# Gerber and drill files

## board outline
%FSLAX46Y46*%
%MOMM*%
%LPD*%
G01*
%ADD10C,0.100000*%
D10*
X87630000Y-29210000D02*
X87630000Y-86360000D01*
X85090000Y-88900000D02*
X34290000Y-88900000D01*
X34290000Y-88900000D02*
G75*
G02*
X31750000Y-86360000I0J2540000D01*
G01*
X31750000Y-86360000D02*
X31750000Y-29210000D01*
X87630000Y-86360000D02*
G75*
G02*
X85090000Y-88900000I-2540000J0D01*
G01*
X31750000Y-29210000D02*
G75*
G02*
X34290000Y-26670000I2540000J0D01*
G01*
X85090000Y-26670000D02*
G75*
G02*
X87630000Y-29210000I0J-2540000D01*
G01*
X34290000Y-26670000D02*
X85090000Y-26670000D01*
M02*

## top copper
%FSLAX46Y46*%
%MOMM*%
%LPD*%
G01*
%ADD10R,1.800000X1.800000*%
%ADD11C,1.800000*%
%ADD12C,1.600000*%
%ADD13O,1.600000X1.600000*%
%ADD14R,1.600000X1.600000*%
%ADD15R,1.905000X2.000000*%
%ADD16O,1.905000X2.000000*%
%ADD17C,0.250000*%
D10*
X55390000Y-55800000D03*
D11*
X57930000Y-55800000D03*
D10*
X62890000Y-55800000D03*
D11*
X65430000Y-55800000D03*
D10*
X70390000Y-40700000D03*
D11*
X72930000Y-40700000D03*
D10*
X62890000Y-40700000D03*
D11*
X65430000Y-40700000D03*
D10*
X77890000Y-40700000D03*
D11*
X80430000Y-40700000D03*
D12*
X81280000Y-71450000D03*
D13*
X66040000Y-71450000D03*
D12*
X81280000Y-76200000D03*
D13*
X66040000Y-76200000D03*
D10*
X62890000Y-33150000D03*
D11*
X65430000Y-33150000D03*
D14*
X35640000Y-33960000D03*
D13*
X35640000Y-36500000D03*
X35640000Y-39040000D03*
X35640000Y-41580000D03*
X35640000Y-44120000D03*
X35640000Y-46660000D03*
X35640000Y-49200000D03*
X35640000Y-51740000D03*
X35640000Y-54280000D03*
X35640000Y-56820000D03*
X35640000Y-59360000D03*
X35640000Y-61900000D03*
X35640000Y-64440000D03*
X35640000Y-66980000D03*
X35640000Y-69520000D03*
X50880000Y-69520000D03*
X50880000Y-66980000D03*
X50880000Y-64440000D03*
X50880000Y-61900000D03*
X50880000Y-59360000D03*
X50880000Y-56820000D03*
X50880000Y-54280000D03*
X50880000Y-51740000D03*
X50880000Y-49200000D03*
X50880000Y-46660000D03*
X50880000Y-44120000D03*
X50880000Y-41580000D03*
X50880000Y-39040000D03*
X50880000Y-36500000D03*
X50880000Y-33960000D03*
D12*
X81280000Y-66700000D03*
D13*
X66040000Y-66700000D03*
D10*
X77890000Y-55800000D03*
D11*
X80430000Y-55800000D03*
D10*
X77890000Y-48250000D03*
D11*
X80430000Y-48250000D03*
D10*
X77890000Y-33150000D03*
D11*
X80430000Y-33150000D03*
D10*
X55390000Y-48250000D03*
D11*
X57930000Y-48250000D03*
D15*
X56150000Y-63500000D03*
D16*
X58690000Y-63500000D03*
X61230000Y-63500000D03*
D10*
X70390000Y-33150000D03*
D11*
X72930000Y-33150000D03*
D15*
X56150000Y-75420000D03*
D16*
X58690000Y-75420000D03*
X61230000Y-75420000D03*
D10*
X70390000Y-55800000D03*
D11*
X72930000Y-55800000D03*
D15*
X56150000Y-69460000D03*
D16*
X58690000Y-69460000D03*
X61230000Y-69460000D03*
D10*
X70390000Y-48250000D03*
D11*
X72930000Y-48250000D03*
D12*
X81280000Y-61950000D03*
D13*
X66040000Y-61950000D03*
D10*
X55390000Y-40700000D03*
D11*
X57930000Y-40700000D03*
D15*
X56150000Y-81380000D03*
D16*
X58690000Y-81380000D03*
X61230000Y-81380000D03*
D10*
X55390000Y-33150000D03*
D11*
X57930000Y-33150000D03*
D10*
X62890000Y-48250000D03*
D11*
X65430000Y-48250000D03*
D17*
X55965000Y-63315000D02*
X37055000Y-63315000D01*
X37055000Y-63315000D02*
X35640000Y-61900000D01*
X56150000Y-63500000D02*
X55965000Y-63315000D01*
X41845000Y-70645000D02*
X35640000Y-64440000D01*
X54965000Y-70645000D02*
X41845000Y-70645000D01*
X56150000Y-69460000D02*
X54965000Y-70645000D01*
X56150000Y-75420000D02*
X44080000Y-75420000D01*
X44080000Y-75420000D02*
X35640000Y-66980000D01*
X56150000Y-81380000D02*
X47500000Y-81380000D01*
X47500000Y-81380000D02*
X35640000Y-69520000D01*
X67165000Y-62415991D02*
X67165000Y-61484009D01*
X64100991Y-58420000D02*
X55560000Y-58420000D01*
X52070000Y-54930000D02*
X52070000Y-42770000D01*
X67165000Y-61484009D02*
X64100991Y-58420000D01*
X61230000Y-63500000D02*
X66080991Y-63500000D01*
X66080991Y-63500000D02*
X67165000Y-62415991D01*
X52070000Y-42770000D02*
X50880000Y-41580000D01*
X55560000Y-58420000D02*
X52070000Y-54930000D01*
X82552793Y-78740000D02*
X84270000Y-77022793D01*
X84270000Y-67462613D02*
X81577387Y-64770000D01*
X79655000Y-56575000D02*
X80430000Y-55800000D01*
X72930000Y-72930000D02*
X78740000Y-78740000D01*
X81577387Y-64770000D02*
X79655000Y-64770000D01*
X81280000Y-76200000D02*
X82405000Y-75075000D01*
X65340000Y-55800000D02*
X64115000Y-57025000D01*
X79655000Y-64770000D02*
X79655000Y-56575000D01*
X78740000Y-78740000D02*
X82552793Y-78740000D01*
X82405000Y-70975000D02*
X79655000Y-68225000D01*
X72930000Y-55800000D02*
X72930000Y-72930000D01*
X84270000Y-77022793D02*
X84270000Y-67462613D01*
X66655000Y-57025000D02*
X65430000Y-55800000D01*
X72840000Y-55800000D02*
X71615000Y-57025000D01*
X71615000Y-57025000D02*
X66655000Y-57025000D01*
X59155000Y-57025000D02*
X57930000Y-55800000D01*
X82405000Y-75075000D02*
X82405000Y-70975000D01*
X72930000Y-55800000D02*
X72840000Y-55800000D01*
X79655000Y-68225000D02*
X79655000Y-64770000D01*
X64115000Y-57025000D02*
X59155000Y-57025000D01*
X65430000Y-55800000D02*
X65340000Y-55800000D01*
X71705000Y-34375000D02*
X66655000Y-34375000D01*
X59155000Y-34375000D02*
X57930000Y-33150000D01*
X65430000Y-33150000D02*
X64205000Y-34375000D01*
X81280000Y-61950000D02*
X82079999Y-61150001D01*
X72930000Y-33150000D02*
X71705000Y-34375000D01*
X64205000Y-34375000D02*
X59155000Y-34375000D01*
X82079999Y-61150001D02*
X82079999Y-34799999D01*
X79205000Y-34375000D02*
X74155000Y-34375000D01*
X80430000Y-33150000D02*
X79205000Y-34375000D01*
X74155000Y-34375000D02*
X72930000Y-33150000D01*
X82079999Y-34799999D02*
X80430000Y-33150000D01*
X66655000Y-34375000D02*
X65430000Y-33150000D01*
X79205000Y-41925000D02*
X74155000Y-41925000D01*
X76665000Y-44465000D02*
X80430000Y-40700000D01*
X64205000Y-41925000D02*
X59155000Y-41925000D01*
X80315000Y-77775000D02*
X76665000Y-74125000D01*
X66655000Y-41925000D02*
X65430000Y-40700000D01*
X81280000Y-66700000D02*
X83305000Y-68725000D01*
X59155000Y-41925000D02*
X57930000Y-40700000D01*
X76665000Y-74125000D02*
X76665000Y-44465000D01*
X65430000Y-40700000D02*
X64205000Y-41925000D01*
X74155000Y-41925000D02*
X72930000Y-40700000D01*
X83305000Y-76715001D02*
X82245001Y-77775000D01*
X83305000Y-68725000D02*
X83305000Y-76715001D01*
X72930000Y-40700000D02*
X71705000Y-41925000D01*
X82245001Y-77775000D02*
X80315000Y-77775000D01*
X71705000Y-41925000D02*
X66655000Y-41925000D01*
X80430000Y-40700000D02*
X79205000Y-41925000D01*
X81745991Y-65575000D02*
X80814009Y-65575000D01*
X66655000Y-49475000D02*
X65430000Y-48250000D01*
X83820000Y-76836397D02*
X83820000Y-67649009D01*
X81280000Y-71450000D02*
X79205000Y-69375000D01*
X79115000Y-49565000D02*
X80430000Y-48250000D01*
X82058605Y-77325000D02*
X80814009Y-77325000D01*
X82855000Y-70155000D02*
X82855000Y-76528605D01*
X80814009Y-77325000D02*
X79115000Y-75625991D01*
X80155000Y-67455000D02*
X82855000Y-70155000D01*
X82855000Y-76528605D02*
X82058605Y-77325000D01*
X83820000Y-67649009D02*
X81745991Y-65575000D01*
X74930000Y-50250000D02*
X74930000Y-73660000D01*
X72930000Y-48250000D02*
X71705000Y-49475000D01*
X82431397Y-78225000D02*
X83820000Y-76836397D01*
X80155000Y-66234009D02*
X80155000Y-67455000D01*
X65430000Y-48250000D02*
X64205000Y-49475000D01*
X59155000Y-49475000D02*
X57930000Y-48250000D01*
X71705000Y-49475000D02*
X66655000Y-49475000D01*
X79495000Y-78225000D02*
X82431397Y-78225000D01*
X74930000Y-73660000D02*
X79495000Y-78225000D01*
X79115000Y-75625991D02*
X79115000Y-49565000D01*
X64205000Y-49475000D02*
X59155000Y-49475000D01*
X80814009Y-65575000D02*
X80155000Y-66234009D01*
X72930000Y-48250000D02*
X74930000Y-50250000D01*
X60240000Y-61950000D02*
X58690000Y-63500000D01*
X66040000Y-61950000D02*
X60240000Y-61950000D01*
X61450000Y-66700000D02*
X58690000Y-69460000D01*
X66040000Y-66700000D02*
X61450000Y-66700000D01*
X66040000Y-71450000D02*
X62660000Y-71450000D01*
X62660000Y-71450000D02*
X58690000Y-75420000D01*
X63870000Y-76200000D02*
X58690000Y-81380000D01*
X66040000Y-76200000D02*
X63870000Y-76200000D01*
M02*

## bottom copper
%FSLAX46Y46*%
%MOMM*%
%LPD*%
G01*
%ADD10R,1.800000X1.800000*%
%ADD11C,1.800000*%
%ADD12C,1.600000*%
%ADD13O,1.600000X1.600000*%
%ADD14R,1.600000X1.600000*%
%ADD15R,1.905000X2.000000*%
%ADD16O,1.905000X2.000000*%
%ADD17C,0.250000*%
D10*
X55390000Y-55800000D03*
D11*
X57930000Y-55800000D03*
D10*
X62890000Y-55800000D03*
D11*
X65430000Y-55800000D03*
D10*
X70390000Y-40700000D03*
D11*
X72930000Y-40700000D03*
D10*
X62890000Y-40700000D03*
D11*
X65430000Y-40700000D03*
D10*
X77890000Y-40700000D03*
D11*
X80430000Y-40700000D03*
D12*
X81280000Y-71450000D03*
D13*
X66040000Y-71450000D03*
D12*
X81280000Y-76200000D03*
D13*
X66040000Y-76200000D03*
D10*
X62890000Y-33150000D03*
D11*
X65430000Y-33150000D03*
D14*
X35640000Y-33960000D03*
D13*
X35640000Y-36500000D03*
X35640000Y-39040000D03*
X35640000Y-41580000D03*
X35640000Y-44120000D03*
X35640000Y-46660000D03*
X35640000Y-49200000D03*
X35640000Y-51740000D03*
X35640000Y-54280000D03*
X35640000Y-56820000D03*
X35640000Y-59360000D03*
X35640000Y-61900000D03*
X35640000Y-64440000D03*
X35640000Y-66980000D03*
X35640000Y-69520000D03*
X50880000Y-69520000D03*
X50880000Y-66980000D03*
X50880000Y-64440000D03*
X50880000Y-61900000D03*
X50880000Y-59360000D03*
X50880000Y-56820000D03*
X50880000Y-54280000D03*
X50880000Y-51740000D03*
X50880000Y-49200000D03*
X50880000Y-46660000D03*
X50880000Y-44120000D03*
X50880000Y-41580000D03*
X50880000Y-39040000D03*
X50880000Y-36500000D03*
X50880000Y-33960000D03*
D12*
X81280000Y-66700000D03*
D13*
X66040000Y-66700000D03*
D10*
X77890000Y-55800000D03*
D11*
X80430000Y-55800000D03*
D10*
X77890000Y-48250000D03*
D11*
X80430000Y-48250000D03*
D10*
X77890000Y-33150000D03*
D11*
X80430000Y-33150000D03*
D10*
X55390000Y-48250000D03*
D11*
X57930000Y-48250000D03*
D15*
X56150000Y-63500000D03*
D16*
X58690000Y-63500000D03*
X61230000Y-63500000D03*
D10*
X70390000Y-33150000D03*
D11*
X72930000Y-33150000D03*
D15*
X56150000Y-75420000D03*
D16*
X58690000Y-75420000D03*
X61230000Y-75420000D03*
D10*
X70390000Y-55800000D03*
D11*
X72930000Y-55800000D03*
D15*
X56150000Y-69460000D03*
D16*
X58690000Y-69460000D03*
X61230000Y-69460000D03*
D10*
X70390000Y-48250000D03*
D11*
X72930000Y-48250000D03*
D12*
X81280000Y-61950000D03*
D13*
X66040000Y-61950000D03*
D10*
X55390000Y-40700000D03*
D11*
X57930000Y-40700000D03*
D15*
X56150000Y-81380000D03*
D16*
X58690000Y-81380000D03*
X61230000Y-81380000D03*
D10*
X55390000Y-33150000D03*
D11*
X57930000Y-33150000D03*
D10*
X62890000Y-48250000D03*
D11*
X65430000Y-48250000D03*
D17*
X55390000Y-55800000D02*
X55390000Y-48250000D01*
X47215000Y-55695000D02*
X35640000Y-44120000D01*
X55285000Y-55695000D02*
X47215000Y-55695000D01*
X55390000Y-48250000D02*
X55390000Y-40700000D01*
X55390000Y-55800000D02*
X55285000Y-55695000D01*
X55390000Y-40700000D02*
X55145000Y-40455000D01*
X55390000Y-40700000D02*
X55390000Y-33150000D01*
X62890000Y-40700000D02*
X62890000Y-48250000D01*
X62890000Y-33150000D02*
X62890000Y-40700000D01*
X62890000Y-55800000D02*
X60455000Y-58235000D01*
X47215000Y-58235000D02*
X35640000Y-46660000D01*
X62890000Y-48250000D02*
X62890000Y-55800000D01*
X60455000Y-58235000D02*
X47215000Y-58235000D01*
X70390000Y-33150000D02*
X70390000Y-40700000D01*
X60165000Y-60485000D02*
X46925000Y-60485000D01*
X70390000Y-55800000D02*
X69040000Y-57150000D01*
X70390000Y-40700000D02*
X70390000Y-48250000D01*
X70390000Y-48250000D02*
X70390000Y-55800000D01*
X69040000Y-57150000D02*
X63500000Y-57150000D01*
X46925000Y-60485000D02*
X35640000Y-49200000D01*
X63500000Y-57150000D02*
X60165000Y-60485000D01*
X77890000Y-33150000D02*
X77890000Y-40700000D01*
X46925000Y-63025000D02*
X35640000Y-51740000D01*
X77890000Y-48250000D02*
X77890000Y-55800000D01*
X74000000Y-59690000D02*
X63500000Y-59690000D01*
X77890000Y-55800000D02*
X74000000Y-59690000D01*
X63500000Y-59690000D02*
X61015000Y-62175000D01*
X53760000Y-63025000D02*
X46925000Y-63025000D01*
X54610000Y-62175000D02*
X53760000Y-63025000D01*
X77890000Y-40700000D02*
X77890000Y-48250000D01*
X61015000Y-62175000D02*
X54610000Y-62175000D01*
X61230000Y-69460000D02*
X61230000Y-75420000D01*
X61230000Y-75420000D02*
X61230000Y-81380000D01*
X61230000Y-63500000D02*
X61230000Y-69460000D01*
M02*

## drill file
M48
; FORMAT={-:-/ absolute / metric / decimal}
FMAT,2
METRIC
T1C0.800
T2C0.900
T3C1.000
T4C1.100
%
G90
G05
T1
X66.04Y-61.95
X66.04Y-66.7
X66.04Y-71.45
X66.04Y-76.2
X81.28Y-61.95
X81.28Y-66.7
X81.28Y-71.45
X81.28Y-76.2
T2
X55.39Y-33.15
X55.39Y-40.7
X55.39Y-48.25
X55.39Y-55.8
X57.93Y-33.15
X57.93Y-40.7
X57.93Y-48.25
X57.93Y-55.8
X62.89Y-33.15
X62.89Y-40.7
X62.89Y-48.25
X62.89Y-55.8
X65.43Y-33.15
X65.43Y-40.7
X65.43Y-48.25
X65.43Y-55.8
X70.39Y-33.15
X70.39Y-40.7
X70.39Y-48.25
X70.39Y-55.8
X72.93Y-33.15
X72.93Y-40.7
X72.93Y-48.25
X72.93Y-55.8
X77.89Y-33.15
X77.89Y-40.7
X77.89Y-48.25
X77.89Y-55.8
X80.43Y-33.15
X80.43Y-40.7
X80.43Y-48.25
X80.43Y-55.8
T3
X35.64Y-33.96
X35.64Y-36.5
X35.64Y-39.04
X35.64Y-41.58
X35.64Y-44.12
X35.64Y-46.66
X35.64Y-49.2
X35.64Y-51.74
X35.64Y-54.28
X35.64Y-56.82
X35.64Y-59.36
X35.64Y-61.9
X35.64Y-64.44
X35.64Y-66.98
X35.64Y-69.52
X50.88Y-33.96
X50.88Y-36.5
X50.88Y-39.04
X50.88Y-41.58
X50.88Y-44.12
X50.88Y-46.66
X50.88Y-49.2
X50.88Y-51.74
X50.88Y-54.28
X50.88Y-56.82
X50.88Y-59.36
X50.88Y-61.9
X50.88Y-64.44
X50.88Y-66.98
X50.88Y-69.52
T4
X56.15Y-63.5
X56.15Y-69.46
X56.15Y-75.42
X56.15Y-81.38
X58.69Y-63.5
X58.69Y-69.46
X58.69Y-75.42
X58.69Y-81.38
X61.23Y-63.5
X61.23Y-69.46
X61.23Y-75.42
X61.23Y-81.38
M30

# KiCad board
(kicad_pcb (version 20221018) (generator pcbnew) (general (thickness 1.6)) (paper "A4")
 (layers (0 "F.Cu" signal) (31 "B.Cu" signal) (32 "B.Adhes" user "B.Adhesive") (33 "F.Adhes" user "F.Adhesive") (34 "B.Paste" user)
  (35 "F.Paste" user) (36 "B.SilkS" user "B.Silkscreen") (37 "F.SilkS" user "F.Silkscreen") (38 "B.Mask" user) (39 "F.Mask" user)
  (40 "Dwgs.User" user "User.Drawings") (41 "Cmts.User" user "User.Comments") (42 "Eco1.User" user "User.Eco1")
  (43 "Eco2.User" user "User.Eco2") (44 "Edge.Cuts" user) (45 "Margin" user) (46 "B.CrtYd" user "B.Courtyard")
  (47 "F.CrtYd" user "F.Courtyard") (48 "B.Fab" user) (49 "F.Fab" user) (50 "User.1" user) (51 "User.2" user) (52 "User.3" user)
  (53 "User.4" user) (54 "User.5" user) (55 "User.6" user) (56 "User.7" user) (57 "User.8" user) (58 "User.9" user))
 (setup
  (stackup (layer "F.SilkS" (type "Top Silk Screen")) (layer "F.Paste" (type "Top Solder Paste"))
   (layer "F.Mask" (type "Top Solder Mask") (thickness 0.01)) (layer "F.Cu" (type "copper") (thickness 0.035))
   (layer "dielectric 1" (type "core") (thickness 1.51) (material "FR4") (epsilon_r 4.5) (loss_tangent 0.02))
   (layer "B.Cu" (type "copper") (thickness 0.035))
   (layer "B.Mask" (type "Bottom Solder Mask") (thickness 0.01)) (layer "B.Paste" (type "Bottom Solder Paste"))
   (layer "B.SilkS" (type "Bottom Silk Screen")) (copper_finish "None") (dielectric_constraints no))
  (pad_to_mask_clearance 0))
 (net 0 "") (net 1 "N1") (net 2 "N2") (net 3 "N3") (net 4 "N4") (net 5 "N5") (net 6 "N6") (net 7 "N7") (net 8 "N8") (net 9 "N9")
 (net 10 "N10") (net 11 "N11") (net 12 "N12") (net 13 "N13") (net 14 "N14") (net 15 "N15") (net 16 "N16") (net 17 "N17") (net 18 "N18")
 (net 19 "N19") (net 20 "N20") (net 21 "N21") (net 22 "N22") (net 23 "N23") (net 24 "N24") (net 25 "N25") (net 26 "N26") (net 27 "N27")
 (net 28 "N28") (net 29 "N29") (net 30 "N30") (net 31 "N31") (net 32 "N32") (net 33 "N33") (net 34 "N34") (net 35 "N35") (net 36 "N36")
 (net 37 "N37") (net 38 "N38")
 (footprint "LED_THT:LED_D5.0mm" (layer "F.Cu") (at 55.39 55.8)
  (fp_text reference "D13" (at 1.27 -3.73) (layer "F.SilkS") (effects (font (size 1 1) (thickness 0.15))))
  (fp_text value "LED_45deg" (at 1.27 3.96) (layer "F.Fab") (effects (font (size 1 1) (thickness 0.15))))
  (pad "1" thru_hole rect (at 0 0) (size 1.8 1.8) (drill 0.9) (layers "*.Cu" "*.Mask") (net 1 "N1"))
  (pad "2" thru_hole circle (at 2.54 0) (size 1.8 1.8) (drill 0.9) (layers "*.Cu" "*.Mask") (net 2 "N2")))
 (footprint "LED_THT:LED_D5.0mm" (layer "F.Cu") (at 62.89 55.8)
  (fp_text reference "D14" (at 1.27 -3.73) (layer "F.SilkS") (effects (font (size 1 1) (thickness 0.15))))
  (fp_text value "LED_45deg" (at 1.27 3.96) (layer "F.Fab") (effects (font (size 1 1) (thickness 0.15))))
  (pad "1" thru_hole rect (at 0 0) (size 1.8 1.8) (drill 0.9) (layers "*.Cu" "*.Mask") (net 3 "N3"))
  (pad "2" thru_hole circle (at 2.54 0) (size 1.8 1.8) (drill 0.9) (layers "*.Cu" "*.Mask") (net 2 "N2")))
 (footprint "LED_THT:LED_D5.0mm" (layer "F.Cu") (at 70.39 40.7)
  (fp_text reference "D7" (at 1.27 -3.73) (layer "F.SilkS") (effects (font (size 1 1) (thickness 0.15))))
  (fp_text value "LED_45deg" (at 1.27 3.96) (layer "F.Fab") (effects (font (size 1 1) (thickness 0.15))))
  (pad "1" thru_hole rect (at 0 0) (size 1.8 1.8) (drill 0.9) (layers "*.Cu" "*.Mask") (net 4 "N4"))
  (pad "2" thru_hole circle (at 2.54 0) (size 1.8 1.8) (drill 0.9) (layers "*.Cu" "*.Mask") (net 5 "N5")))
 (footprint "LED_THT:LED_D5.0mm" (layer "F.Cu") (at 62.89 40.7)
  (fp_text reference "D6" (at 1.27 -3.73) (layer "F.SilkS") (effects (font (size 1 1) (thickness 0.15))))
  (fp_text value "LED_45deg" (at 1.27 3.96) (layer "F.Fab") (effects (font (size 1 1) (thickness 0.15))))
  (pad "1" thru_hole rect (at 0 0) (size 1.8 1.8) (drill 0.9) (layers "*.Cu" "*.Mask") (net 3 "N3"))
  (pad "2" thru_hole circle (at 2.54 0) (size 1.8 1.8) (drill 0.9) (layers "*.Cu" "*.Mask") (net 5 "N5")))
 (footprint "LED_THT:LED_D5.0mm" (layer "F.Cu") (at 77.89 40.7)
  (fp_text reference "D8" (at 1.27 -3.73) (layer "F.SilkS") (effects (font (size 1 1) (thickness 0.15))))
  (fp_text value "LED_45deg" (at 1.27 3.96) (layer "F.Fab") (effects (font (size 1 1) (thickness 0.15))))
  (pad "1" thru_hole rect (at 0 0) (size 1.8 1.8) (drill 0.9) (layers "*.Cu" "*.Mask") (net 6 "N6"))
  (pad "2" thru_hole circle (at 2.54 0) (size 1.8 1.8) (drill 0.9) (layers "*.Cu" "*.Mask") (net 5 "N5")))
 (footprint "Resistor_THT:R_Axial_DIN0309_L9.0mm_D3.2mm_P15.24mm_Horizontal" (layer "F.Cu") (at 81.28 71.45 180)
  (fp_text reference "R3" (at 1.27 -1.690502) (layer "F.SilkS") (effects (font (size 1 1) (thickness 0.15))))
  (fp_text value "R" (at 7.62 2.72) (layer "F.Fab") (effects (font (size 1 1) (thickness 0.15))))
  (pad "1" thru_hole circle (at 0 0 180) (size 1.6 1.6) (drill 0.8) (layers "*.Cu" "*.Mask") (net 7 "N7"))
  (pad "2" thru_hole oval (at 15.24 0 180) (size 1.6 1.6) (drill 0.8) (layers "*.Cu" "*.Mask") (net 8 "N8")))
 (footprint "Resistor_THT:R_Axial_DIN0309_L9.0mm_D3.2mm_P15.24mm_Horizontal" (layer "F.Cu") (at 81.28 76.2 180)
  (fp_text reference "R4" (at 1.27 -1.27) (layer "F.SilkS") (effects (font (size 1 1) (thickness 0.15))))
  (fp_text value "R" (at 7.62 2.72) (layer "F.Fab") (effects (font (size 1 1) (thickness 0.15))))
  (pad "1" thru_hole circle (at 0 0 180) (size 1.6 1.6) (drill 0.8) (layers "*.Cu" "*.Mask") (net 2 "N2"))
  (pad "2" thru_hole oval (at 15.24 0 180) (size 1.6 1.6) (drill 0.8) (layers "*.Cu" "*.Mask") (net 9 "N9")))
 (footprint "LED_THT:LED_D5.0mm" (layer "F.Cu") (at 62.89 33.15)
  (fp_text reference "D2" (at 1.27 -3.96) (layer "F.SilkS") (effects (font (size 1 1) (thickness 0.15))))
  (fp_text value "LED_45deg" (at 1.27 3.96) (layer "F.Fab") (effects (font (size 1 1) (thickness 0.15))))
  (pad "1" thru_hole rect (at 0 0) (size 1.8 1.8) (drill 0.9) (layers "*.Cu" "*.Mask") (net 3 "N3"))
  (pad "2" thru_hole circle (at 2.54 0) (size 1.8 1.8) (drill 0.9) (layers "*.Cu" "*.Mask") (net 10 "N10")))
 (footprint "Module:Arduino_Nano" (layer "F.Cu") (at 35.64 33.96)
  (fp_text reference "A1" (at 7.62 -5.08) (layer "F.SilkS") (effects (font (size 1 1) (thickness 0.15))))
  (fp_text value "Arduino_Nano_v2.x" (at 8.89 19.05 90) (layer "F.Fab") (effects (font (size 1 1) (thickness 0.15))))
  (pad "1" thru_hole rect (at 0 0) (size 1.6 1.6) (drill 1) (layers "*.Cu" "*.Mask") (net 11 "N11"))
  (pad "2" thru_hole oval (at 0 2.54) (size 1.6 1.6) (drill 1) (layers "*.Cu" "*.Mask") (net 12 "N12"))
  (pad "3" thru_hole oval (at 0 5.08) (size 1.6 1.6) (drill 1) (layers "*.Cu" "*.Mask") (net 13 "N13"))
  (pad "4" thru_hole oval (at 0 7.62) (size 1.6 1.6) (drill 1) (layers "*.Cu" "*.Mask") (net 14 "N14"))
  (pad "5" thru_hole oval (at 0 10.16) (size 1.6 1.6) (drill 1) (layers "*.Cu" "*.Mask") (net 1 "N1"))
  (pad "6" thru_hole oval (at 0 12.7) (size 1.6 1.6) (drill 1) (layers "*.Cu" "*.Mask") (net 3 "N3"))
  (pad "7" thru_hole oval (at 0 15.24) (size 1.6 1.6) (drill 1) (layers "*.Cu" "*.Mask") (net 4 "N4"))
  (pad "8" thru_hole oval (at 0 17.78) (size 1.6 1.6) (drill 1) (layers "*.Cu" "*.Mask") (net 6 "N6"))
  (pad "9" thru_hole oval (at 0 20.32) (size 1.6 1.6) (drill 1) (layers "*.Cu" "*.Mask") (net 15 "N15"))
  (pad "10" thru_hole oval (at 0 22.86) (size 1.6 1.6) (drill 1) (layers "*.Cu" "*.Mask") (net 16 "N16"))
  (pad "11" thru_hole oval (at 0 25.4) (size 1.6 1.6) (drill 1) (layers "*.Cu" "*.Mask") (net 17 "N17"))
  (pad "12" thru_hole oval (at 0 27.94) (size 1.6 1.6) (drill 1) (layers "*.Cu" "*.Mask") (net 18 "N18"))
  (pad "13" thru_hole oval (at 0 30.48) (size 1.6 1.6) (drill 1) (layers "*.Cu" "*.Mask") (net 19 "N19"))
  (pad "14" thru_hole oval (at 0 33.02) (size 1.6 1.6) (drill 1) (layers "*.Cu" "*.Mask") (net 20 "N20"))
  (pad "15" thru_hole oval (at 0 35.56) (size 1.6 1.6) (drill 1) (layers "*.Cu" "*.Mask") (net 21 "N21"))
  (pad "16" thru_hole oval (at 15.24 35.56) (size 1.6 1.6) (drill 1) (layers "*.Cu" "*.Mask") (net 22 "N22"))
  (pad "17" thru_hole oval (at 15.24 33.02) (size 1.6 1.6) (drill 1) (layers "*.Cu" "*.Mask") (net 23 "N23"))
  (pad "18" thru_hole oval (at 15.24 30.48) (size 1.6 1.6) (drill 1) (layers "*.Cu" "*.Mask") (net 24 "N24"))
  (pad "19" thru_hole oval (at 15.24 27.94) (size 1.6 1.6) (drill 1) (layers "*.Cu" "*.Mask") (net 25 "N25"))
  (pad "20" thru_hole oval (at 15.24 25.4) (size 1.6 1.6) (drill 1) (layers "*.Cu" "*.Mask") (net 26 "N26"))
  (pad "21" thru_hole oval (at 15.24 22.86) (size 1.6 1.6) (drill 1) (layers "*.Cu" "*.Mask") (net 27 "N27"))
  (pad "22" thru_hole oval (at 15.24 20.32) (size 1.6 1.6) (drill 1) (layers "*.Cu" "*.Mask") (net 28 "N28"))
  (pad "23" thru_hole oval (at 15.24 17.78) (size 1.6 1.6) (drill 1) (layers "*.Cu" "*.Mask") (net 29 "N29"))
  (pad "24" thru_hole oval (at 15.24 15.24) (size 1.6 1.6) (drill 1) (layers "*.Cu" "*.Mask") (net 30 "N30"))
  (pad "25" thru_hole oval (at 15.24 12.7) (size 1.6 1.6) (drill 1) (layers "*.Cu" "*.Mask") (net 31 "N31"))
  (pad "26" thru_hole oval (at 15.24 10.16) (size 1.6 1.6) (drill 1) (layers "*.Cu" "*.Mask") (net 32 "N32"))
  (pad "27" thru_hole oval (at 15.24 7.62) (size 1.6 1.6) (drill 1) (layers "*.Cu" "*.Mask") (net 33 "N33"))
  (pad "28" thru_hole oval (at 15.24 5.08) (size 1.6 1.6) (drill 1) (layers "*.Cu" "*.Mask") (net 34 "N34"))
  (pad "29" thru_hole oval (at 15.24 2.54) (size 1.6 1.6) (drill 1) (layers "*.Cu" "*.Mask") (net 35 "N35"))
  (pad "30" thru_hole oval (at 15.24 0) (size 1.6 1.6) (drill 1) (layers "*.Cu" "*.Mask") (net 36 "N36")))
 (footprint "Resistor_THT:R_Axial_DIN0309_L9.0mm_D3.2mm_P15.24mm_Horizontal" (layer "F.Cu") (at 81.28 66.7 180)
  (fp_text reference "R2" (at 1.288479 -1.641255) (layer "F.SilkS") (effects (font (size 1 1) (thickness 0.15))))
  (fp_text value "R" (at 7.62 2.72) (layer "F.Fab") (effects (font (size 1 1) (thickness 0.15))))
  (pad "1" thru_hole circle (at 0 0 180) (size 1.6 1.6) (drill 0.8) (layers "*.Cu" "*.Mask") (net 5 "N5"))
  (pad "2" thru_hole oval (at 15.24 0 180) (size 1.6 1.6) (drill 0.8) (layers "*.Cu" "*.Mask") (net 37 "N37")))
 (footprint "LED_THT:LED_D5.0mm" (layer "F.Cu") (at 77.89 55.8)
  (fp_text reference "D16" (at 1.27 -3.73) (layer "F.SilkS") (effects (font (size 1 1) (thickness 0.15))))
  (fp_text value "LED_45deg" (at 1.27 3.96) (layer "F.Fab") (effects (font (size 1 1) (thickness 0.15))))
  (pad "1" thru_hole rect (at 0 0) (size 1.8 1.8) (drill 0.9) (layers "*.Cu" "*.Mask") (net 6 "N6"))
  (pad "2" thru_hole circle (at 2.54 0) (size 1.8 1.8) (drill 0.9) (layers "*.Cu" "*.Mask") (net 2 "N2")))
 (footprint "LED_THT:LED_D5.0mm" (layer "F.Cu") (at 77.89 48.25)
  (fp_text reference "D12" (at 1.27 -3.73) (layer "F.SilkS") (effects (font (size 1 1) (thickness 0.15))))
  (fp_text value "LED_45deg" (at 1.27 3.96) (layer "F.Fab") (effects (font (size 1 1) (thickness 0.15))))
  (pad "1" thru_hole rect (at 0 0) (size 1.8 1.8) (drill 0.9) (layers "*.Cu" "*.Mask") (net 6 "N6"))
  (pad "2" thru_hole circle (at 2.54 0) (size 1.8 1.8) (drill 0.9) (layers "*.Cu" "*.Mask") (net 7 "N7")))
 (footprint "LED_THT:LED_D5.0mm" (layer "F.Cu") (at 77.89 33.15)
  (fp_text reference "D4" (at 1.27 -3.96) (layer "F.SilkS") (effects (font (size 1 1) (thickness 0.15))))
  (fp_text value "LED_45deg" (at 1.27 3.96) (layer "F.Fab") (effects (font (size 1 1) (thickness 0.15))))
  (pad "1" thru_hole rect (at 0 0) (size 1.8 1.8) (drill 0.9) (layers "*.Cu" "*.Mask") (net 6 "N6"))
  (pad "2" thru_hole circle (at 2.54 0) (size 1.8 1.8) (drill 0.9) (layers "*.Cu" "*.Mask") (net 10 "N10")))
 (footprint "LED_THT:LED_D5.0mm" (layer "F.Cu") (at 55.39 48.25)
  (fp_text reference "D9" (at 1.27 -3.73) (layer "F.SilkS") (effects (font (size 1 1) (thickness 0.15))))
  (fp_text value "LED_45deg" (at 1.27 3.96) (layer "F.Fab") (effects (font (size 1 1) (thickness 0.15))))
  (pad "1" thru_hole rect (at 0 0) (size 1.8 1.8) (drill 0.9) (layers "*.Cu" "*.Mask") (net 1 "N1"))
  (pad "2" thru_hole circle (at 2.54 0) (size 1.8 1.8) (drill 0.9) (layers "*.Cu" "*.Mask") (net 7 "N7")))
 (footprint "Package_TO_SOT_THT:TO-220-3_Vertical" (layer "F.Cu") (at 56.15 63.5)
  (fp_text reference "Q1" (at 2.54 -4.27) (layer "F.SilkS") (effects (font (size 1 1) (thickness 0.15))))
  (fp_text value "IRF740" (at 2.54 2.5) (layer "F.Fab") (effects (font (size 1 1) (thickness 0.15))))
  (pad "1" thru_hole rect (at 0 0) (size 1.905 2) (drill 1.1) (layers "*.Cu" "*.Mask") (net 18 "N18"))
  (pad "2" thru_hole oval (at 2.54 0) (size 1.905 2) (drill 1.1) (layers "*.Cu" "*.Mask") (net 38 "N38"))
  (pad "3" thru_hole oval (at 5.08 0) (size 1.905 2) (drill 1.1) (layers "*.Cu" "*.Mask") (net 33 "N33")))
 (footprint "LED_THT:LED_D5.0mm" (layer "F.Cu") (at 70.39 33.15)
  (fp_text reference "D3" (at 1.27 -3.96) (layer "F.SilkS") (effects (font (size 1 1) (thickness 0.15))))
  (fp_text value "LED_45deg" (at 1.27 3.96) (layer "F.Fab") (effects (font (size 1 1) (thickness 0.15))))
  (pad "1" thru_hole rect (at 0 0) (size 1.8 1.8) (drill 0.9) (layers "*.Cu" "*.Mask") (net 4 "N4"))
  (pad "2" thru_hole circle (at 2.54 0) (size 1.8 1.8) (drill 0.9) (layers "*.Cu" "*.Mask") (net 10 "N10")))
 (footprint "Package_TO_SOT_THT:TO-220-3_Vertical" (layer "F.Cu") (at 56.15 75.42)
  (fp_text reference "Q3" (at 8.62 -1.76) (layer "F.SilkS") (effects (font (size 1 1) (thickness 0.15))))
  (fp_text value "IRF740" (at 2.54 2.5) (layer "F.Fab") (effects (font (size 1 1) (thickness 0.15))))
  (pad "1" thru_hole rect (at 0 0) (size 1.905 2) (drill 1.1) (layers "*.Cu" "*.Mask") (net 20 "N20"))
  (pad "2" thru_hole oval (at 2.54 0) (size 1.905 2) (drill 1.1) (layers "*.Cu" "*.Mask") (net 8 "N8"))
  (pad "3" thru_hole oval (at 5.08 0) (size 1.905 2) (drill 1.1) (layers "*.Cu" "*.Mask") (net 33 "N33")))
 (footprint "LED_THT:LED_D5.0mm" (layer "F.Cu") (at 70.39 55.8)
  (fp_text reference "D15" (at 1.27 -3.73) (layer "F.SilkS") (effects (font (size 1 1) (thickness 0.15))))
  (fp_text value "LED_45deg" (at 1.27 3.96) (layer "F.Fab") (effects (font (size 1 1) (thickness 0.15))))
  (pad "1" thru_hole rect (at 0 0) (size 1.8 1.8) (drill 0.9) (layers "*.Cu" "*.Mask") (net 4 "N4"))
  (pad "2" thru_hole circle (at 2.54 0) (size 1.8 1.8) (drill 0.9) (layers "*.Cu" "*.Mask") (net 2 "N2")))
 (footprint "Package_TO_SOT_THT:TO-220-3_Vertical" (layer "F.Cu") (at 56.15 69.46)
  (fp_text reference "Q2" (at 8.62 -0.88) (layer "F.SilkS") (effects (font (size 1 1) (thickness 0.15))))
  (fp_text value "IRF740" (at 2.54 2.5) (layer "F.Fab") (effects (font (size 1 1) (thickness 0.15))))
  (pad "1" thru_hole rect (at 0 0) (size 1.905 2) (drill 1.1) (layers "*.Cu" "*.Mask") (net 19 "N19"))
  (pad "2" thru_hole oval (at 2.54 0) (size 1.905 2) (drill 1.1) (layers "*.Cu" "*.Mask") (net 37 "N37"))
  (pad "3" thru_hole oval (at 5.08 0) (size 1.905 2) (drill 1.1) (layers "*.Cu" "*.Mask") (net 33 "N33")))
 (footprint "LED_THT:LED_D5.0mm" (layer "F.Cu") (at 70.39 48.25)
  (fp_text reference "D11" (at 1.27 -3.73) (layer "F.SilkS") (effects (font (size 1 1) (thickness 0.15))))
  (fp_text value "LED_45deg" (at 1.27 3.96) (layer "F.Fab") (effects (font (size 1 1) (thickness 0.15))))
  (pad "1" thru_hole rect (at 0 0) (size 1.8 1.8) (drill 0.9) (layers "*.Cu" "*.Mask") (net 4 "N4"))
  (pad "2" thru_hole circle (at 2.54 0) (size 1.8 1.8) (drill 0.9) (layers "*.Cu" "*.Mask") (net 7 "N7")))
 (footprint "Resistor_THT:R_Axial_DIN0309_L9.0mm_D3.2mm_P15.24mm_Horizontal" (layer "F.Cu") (at 81.28 61.95 180)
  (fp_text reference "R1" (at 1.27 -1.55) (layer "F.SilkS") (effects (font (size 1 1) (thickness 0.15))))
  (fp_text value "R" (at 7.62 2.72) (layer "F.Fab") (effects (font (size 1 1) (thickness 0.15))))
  (pad "1" thru_hole circle (at 0 0 180) (size 1.6 1.6) (drill 0.8) (layers "*.Cu" "*.Mask") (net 10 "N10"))
  (pad "2" thru_hole oval (at 15.24 0 180) (size 1.6 1.6) (drill 0.8) (layers "*.Cu" "*.Mask") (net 38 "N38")))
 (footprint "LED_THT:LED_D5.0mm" (layer "F.Cu") (at 55.39 40.7)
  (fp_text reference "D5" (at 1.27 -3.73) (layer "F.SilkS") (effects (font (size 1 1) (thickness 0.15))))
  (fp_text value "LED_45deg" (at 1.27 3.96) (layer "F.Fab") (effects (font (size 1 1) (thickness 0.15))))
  (pad "1" thru_hole rect (at 0 0) (size 1.8 1.8) (drill 0.9) (layers "*.Cu" "*.Mask") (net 1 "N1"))
  (pad "2" thru_hole circle (at 2.54 0) (size 1.8 1.8) (drill 0.9) (layers "*.Cu" "*.Mask") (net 5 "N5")))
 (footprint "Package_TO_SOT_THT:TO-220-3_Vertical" (layer "F.Cu") (at 56.15 81.38)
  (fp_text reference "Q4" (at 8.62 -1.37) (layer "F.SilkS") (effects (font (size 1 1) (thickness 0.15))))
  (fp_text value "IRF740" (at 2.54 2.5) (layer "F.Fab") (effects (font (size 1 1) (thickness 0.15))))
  (pad "1" thru_hole rect (at 0 0) (size 1.905 2) (drill 1.1) (layers "*.Cu" "*.Mask") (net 21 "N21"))
  (pad "2" thru_hole oval (at 2.54 0) (size 1.905 2) (drill 1.1) (layers "*.Cu" "*.Mask") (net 9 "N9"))
  (pad "3" thru_hole oval (at 5.08 0) (size 1.905 2) (drill 1.1) (layers "*.Cu" "*.Mask") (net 33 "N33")))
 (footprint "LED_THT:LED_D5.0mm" (layer "F.Cu") (at 55.39 33.15)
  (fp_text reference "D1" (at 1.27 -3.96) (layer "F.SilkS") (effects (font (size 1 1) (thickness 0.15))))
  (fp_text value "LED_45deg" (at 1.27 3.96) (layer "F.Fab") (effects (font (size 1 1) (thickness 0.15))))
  (pad "1" thru_hole rect (at 0 0) (size 1.8 1.8) (drill 0.9) (layers "*.Cu" "*.Mask") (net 1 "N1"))
  (pad "2" thru_hole circle (at 2.54 0) (size 1.8 1.8) (drill 0.9) (layers "*.Cu" "*.Mask") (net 10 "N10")))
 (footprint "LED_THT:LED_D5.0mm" (layer "F.Cu") (at 62.89 48.25)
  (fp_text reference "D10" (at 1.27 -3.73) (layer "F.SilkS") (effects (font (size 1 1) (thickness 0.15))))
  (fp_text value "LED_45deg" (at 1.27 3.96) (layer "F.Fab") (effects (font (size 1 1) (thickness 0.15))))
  (pad "1" thru_hole rect (at 0 0) (size 1.8 1.8) (drill 0.9) (layers "*.Cu" "*.Mask") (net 3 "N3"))
  (pad "2" thru_hole circle (at 2.54 0) (size 1.8 1.8) (drill 0.9) (layers "*.Cu" "*.Mask") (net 7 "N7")))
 (gr_line (start 87.63 29.21) (end 87.63 86.36) (stroke (width 0.1) (type default)) (layer "Edge.Cuts"))
 (gr_line (start 85.09 88.9) (end 34.29 88.9) (stroke (width 0.1) (type default)) (layer "Edge.Cuts"))
 (gr_arc (start 34.29 88.9) (mid 32.493949 88.156051) (end 31.75 86.36) (stroke (width 0.1) (type default)) (layer "Edge.Cuts"))
 (gr_line (start 31.75 86.36) (end 31.75 29.21) (stroke (width 0.1) (type default)) (layer "Edge.Cuts"))
 (gr_arc (start 87.63 86.36) (mid 86.886051 88.156051) (end 85.09 88.9) (stroke (width 0.1) (type default)) (layer "Edge.Cuts"))
 (gr_arc (start 31.75 29.21) (mid 32.493949 27.413949) (end 34.29 26.67) (stroke (width 0.1) (type default)) (layer "Edge.Cuts"))
 (gr_arc (start 85.09 26.67) (mid 86.886051 27.413949) (end 87.63 29.21) (stroke (width 0.1) (type default)) (layer "Edge.Cuts"))
 (gr_line (start 34.29 26.67) (end 85.09 26.67) (stroke (width 0.1) (type default)) (layer "Edge.Cuts"))
 (segment (start 55.39 55.8) (end 55.39 48.25) (width 0.25) (layer "B.Cu") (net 1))
 (segment (start 47.215 55.695) (end 35.64 44.12) (width 0.25) (layer "B.Cu") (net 1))
 (segment (start 55.285 55.695) (end 47.215 55.695) (width 0.25) (layer "B.Cu") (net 1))
 (segment (start 55.39 48.25) (end 55.39 40.7) (width 0.25) (layer "B.Cu") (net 1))
 (segment (start 55.39 55.8) (end 55.285 55.695) (width 0.25) (layer "B.Cu") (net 1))
 (segment (start 55.39 40.7) (end 55.145 40.455) (width 0.25) (layer "B.Cu") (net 1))
 (segment (start 55.39 40.7) (end 55.39 33.15) (width 0.25) (layer "B.Cu") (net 1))
 (segment (start 62.89 40.7) (end 62.89 48.25) (width 0.25) (layer "B.Cu") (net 3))
 (segment (start 62.89 33.15) (end 62.89 40.7) (width 0.25) (layer "B.Cu") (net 3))
 (segment (start 62.89 55.8) (end 60.455 58.235) (width 0.25) (layer "B.Cu") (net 3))
 (segment (start 47.215 58.235) (end 35.64 46.66) (width 0.25) (layer "B.Cu") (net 3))
 (segment (start 62.89 48.25) (end 62.89 55.8) (width 0.25) (layer "B.Cu") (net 3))
 (segment (start 60.455 58.235) (end 47.215 58.235) (width 0.25) (layer "B.Cu") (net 3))
 (segment (start 70.39 33.15) (end 70.39 40.7) (width 0.25) (layer "B.Cu") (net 4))
 (segment (start 60.165 60.485) (end 46.925 60.485) (width 0.25) (layer "B.Cu") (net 4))
 (segment (start 70.39 55.8) (end 69.04 57.15) (width 0.25) (layer "B.Cu") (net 4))
 (segment (start 70.39 40.7) (end 70.39 48.25) (width 0.25) (layer "B.Cu") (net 4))
 (segment (start 70.39 48.25) (end 70.39 55.8) (width 0.25) (layer "B.Cu") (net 4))
 (segment (start 69.04 57.15) (end 63.5 57.15) (width 0.25) (layer "B.Cu") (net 4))
 (segment (start 46.925 60.485) (end 35.64 49.2) (width 0.25) (layer "B.Cu") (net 4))
 (segment (start 63.5 57.15) (end 60.165 60.485) (width 0.25) (layer "B.Cu") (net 4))
 (segment (start 77.89 33.15) (end 77.89 40.7) (width 0.25) (layer "B.Cu") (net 6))
 (segment (start 46.925 63.025) (end 35.64 51.74) (width 0.25) (layer "B.Cu") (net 6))
 (segment (start 77.89 48.25) (end 77.89 55.8) (width 0.25) (layer "B.Cu") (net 6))
 (segment (start 74 59.69) (end 63.5 59.69) (width 0.25) (layer "B.Cu") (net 6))
 (segment (start 77.89 55.8) (end 74 59.69) (width 0.25) (layer "B.Cu") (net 6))
 (segment (start 63.5 59.69) (end 61.015 62.175) (width 0.25) (layer "B.Cu") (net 6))
 (segment (start 53.76 63.025) (end 46.925 63.025) (width 0.25) (layer "B.Cu") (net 6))
 (segment (start 54.61 62.175) (end 53.76 63.025) (width 0.25) (layer "B.Cu") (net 6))
 (segment (start 77.89 40.7) (end 77.89 48.25) (width 0.25) (layer "B.Cu") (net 6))
 (segment (start 61.015 62.175) (end 54.61 62.175) (width 0.25) (layer "B.Cu") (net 6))
 (segment (start 55.965 63.315) (end 37.055 63.315) (width 0.25) (layer "F.Cu") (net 18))
 (segment (start 37.055 63.315) (end 35.64 61.9) (width 0.25) (layer "F.Cu") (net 18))
 (segment (start 56.15 63.5) (end 55.965 63.315) (width 0.25) (layer "F.Cu") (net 18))
 (segment (start 41.845 70.645) (end 35.64 64.44) (width 0.25) (layer "F.Cu") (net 19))
 (segment (start 54.965 70.645) (end 41.845 70.645) (width 0.25) (layer "F.Cu") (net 19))
 (segment (start 56.15 69.46) (end 54.965 70.645) (width 0.25) (layer "F.Cu") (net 19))
 (segment (start 56.15 75.42) (end 44.08 75.42) (width 0.25) (layer "F.Cu") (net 20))
 (segment (start 44.08 75.42) (end 35.64 66.98) (width 0.25) (layer "F.Cu") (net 20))
 (segment (start 56.15 81.38) (end 47.5 81.38) (width 0.25) (layer "F.Cu") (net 21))
 (segment (start 47.5 81.38) (end 35.64 69.52) (width 0.25) (layer "F.Cu") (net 21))
 (segment (start 67.165 62.415991) (end 67.165 61.484009) (width 0.25) (layer "F.Cu") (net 33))
 (segment (start 64.100991 58.42) (end 55.56 58.42) (width 0.25) (layer "F.Cu") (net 33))
 (segment (start 52.07 54.93) (end 52.07 42.77) (width 0.25) (layer "F.Cu") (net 33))
 (segment (start 67.165 61.484009) (end 64.100991 58.42) (width 0.25) (layer "F.Cu") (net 33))
 (segment (start 61.23 63.5) (end 66.080991 63.5) (width 0.25) (layer "F.Cu") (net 33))
 (segment (start 66.080991 63.5) (end 67.165 62.415991) (width 0.25) (layer "F.Cu") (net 33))
 (segment (start 52.07 42.77) (end 50.88 41.58) (width 0.25) (layer "F.Cu") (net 33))
 (segment (start 55.56 58.42) (end 52.07 54.93) (width 0.25) (layer "F.Cu") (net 33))
 (segment (start 61.23 69.46) (end 61.23 75.42) (width 0.25) (layer "B.Cu") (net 33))
 (segment (start 61.23 75.42) (end 61.23 81.38) (width 0.25) (layer "B.Cu") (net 33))
 (segment (start 61.23 63.5) (end 61.23 69.46) (width 0.25) (layer "B.Cu") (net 33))
 (segment (start 82.552793 78.74) (end 84.27 77.022793) (width 0.25) (layer "F.Cu") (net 2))
 (segment (start 84.27 67.462613) (end 81.577387 64.77) (width 0.25) (layer "F.Cu") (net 2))
 (segment (start 79.655 56.575) (end 80.43 55.8) (width 0.25) (layer "F.Cu") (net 2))
 (segment (start 72.93 72.93) (end 78.74 78.74) (width 0.25) (layer "F.Cu") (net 2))
 (segment (start 81.577387 64.77) (end 79.655 64.77) (width 0.25) (layer "F.Cu") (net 2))
 (segment (start 81.28 76.2) (end 82.405 75.075) (width 0.25) (layer "F.Cu") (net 2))
 (segment (start 65.34 55.8) (end 64.115 57.025) (width 0.25) (layer "F.Cu") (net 2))
 (segment (start 79.655 64.77) (end 79.655 56.575) (width 0.25) (layer "F.Cu") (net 2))
 (segment (start 78.74 78.74) (end 82.552793 78.74) (width 0.25) (layer "F.Cu") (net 2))
 (segment (start 82.405 70.975) (end 79.655 68.225) (width 0.25) (layer "F.Cu") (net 2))
 (segment (start 72.93 55.8) (end 72.93 72.93) (width 0.25) (layer "F.Cu") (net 2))
 (segment (start 84.27 77.022793) (end 84.27 67.462613) (width 0.25) (layer "F.Cu") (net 2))
 (segment (start 66.655 57.025) (end 65.43 55.8) (width 0.25) (layer "F.Cu") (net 2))
 (segment (start 72.84 55.8) (end 71.615 57.025) (width 0.25) (layer "F.Cu") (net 2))
 (segment (start 71.615 57.025) (end 66.655 57.025) (width 0.25) (layer "F.Cu") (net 2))
 (segment (start 59.155 57.025) (end 57.93 55.8) (width 0.25) (layer "F.Cu") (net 2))
 (segment (start 82.405 75.075) (end 82.405 70.975) (width 0.25) (layer "F.Cu") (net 2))
 (segment (start 72.93 55.8) (end 72.84 55.8) (width 0.25) (layer "F.Cu") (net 2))
 (segment (start 79.655 68.225) (end 79.655 64.77) (width 0.25) (layer "F.Cu") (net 2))
 (segment (start 64.115 57.025) (end 59.155 57.025) (width 0.25) (layer "F.Cu") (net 2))
 (segment (start 65.43 55.8) (end 65.34 55.8) (width 0.25) (layer "F.Cu") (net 2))
 (segment (start 71.705 34.375) (end 66.655 34.375) (width 0.25) (layer "F.Cu") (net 10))
 (segment (start 59.155 34.375) (end 57.93 33.15) (width 0.25) (layer "F.Cu") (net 10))
 (segment (start 65.43 33.15) (end 64.205 34.375) (width 0.25) (layer "F.Cu") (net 10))
 (segment (start 81.28 61.95) (end 82.079999 61.150001) (width 0.25) (layer "F.Cu") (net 10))
 (segment (start 72.93 33.15) (end 71.705 34.375) (width 0.25) (layer "F.Cu") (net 10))
 (segment (start 64.205 34.375) (end 59.155 34.375) (width 0.25) (layer "F.Cu") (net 10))
 (segment (start 82.079999 61.150001) (end 82.079999 34.799999) (width 0.25) (layer "F.Cu") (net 10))
 (segment (start 79.205 34.375) (end 74.155 34.375) (width 0.25) (layer "F.Cu") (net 10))
 (segment (start 80.43 33.15) (end 79.205 34.375) (width 0.25) (layer "F.Cu") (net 10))
 (segment (start 74.155 34.375) (end 72.93 33.15) (width 0.25) (layer "F.Cu") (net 10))
 (segment (start 82.079999 34.799999) (end 80.43 33.15) (width 0.25) (layer "F.Cu") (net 10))
 (segment (start 66.655 34.375) (end 65.43 33.15) (width 0.25) (layer "F.Cu") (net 10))
 (segment (start 79.205 41.925) (end 74.155 41.925) (width 0.25) (layer "F.Cu") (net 5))
 (segment (start 76.665 44.465) (end 80.43 40.7) (width 0.25) (layer "F.Cu") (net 5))
 (segment (start 64.205 41.925) (end 59.155 41.925) (width 0.25) (layer "F.Cu") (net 5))
 (segment (start 80.315 77.775) (end 76.665 74.125) (width 0.25) (layer "F.Cu") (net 5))
 (segment (start 66.655 41.925) (end 65.43 40.7) (width 0.25) (layer "F.Cu") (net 5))
 (segment (start 81.28 66.7) (end 83.305 68.725) (width 0.25) (layer "F.Cu") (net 5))
 (segment (start 59.155 41.925) (end 57.93 40.7) (width 0.25) (layer "F.Cu") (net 5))
 (segment (start 76.665 74.125) (end 76.665 44.465) (width 0.25) (layer "F.Cu") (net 5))
 (segment (start 65.43 40.7) (end 64.205 41.925) (width 0.25) (layer "F.Cu") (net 5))
 (segment (start 74.155 41.925) (end 72.93 40.7) (width 0.25) (layer "F.Cu") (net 5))
 (segment (start 83.305 76.715001) (end 82.245001 77.775) (width 0.25) (layer "F.Cu") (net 5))
 (segment (start 83.305 68.725) (end 83.305 76.715001) (width 0.25) (layer "F.Cu") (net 5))
 (segment (start 72.93 40.7) (end 71.705 41.925) (width 0.25) (layer "F.Cu") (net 5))
 (segment (start 82.245001 77.775) (end 80.315 77.775) (width 0.25) (layer "F.Cu") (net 5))
 (segment (start 71.705 41.925) (end 66.655 41.925) (width 0.25) (layer "F.Cu") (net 5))
 (segment (start 80.43 40.7) (end 79.205 41.925) (width 0.25) (layer "F.Cu") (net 5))
 (segment (start 81.745991 65.575) (end 80.814009 65.575) (width 0.25) (layer "F.Cu") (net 7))
 (segment (start 66.655 49.475) (end 65.43 48.25) (width 0.25) (layer "F.Cu") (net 7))
 (segment (start 83.82 76.836397) (end 83.82 67.649009) (width 0.25) (layer "F.Cu") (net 7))
 (segment (start 81.28 71.45) (end 79.205 69.375) (width 0.25) (layer "F.Cu") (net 7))
 (segment (start 79.115 49.565) (end 80.43 48.25) (width 0.25) (layer "F.Cu") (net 7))
 (segment (start 82.058605 77.325) (end 80.814009 77.325) (width 0.25) (layer "F.Cu") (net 7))
 (segment (start 82.855 70.155) (end 82.855 76.528605) (width 0.25) (layer "F.Cu") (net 7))
 (segment (start 80.814009 77.325) (end 79.115 75.625991) (width 0.25) (layer "F.Cu") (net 7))
 (segment (start 80.155 67.455) (end 82.855 70.155) (width 0.25) (layer "F.Cu") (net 7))
 (segment (start 82.855 76.528605) (end 82.058605 77.325) (width 0.25) (layer "F.Cu") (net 7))
 (segment (start 83.82 67.649009) (end 81.745991 65.575) (width 0.25) (layer "F.Cu") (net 7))
 (segment (start 74.93 50.25) (end 74.93 73.66) (width 0.25) (layer "F.Cu") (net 7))
 (segment (start 72.93 48.25) (end 71.705 49.475) (width 0.25) (layer "F.Cu") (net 7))
 (segment (start 82.431397 78.225) (end 83.82 76.836397) (width 0.25) (layer "F.Cu") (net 7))
 (segment (start 80.155 66.234009) (end 80.155 67.455) (width 0.25) (layer "F.Cu") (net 7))
 (segment (start 65.43 48.25) (end 64.205 49.475) (width 0.25) (layer "F.Cu") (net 7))
 (segment (start 59.155 49.475) (end 57.93 48.25) (width 0.25) (layer "F.Cu") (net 7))
 (segment (start 71.705 49.475) (end 66.655 49.475) (width 0.25) (layer "F.Cu") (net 7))
 (segment (start 79.495 78.225) (end 82.431397 78.225) (width 0.25) (layer "F.Cu") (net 7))
 (segment (start 74.93 73.66) (end 79.495 78.225) (width 0.25) (layer "F.Cu") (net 7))
 (segment (start 79.115 75.625991) (end 79.115 49.565) (width 0.25) (layer "F.Cu") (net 7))
 (segment (start 64.205 49.475) (end 59.155 49.475) (width 0.25) (layer "F.Cu") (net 7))
 (segment (start 80.814009 65.575) (end 80.155 66.234009) (width 0.25) (layer "F.Cu") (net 7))
 (segment (start 72.93 48.25) (end 74.93 50.25) (width 0.25) (layer "F.Cu") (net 7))
 (segment (start 60.24 61.95) (end 58.69 63.5) (width 0.25) (layer "F.Cu") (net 38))
 (segment (start 66.04 61.95) (end 60.24 61.95) (width 0.25) (layer "F.Cu") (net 38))
 (segment (start 61.45 66.7) (end 58.69 69.46) (width 0.25) (layer "F.Cu") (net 37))
 (segment (start 66.04 66.7) (end 61.45 66.7) (width 0.25) (layer "F.Cu") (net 37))
 (segment (start 66.04 71.45) (end 62.66 71.45) (width 0.25) (layer "F.Cu") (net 8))
 (segment (start 62.66 71.45) (end 58.69 75.42) (width 0.25) (layer "F.Cu") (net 8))
 (segment (start 63.87 76.2) (end 58.69 81.38) (width 0.25) (layer "F.Cu") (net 9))
 (segment (start 66.04 76.2) (end 63.87 76.2) (width 0.25) (layer "F.Cu") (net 9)))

